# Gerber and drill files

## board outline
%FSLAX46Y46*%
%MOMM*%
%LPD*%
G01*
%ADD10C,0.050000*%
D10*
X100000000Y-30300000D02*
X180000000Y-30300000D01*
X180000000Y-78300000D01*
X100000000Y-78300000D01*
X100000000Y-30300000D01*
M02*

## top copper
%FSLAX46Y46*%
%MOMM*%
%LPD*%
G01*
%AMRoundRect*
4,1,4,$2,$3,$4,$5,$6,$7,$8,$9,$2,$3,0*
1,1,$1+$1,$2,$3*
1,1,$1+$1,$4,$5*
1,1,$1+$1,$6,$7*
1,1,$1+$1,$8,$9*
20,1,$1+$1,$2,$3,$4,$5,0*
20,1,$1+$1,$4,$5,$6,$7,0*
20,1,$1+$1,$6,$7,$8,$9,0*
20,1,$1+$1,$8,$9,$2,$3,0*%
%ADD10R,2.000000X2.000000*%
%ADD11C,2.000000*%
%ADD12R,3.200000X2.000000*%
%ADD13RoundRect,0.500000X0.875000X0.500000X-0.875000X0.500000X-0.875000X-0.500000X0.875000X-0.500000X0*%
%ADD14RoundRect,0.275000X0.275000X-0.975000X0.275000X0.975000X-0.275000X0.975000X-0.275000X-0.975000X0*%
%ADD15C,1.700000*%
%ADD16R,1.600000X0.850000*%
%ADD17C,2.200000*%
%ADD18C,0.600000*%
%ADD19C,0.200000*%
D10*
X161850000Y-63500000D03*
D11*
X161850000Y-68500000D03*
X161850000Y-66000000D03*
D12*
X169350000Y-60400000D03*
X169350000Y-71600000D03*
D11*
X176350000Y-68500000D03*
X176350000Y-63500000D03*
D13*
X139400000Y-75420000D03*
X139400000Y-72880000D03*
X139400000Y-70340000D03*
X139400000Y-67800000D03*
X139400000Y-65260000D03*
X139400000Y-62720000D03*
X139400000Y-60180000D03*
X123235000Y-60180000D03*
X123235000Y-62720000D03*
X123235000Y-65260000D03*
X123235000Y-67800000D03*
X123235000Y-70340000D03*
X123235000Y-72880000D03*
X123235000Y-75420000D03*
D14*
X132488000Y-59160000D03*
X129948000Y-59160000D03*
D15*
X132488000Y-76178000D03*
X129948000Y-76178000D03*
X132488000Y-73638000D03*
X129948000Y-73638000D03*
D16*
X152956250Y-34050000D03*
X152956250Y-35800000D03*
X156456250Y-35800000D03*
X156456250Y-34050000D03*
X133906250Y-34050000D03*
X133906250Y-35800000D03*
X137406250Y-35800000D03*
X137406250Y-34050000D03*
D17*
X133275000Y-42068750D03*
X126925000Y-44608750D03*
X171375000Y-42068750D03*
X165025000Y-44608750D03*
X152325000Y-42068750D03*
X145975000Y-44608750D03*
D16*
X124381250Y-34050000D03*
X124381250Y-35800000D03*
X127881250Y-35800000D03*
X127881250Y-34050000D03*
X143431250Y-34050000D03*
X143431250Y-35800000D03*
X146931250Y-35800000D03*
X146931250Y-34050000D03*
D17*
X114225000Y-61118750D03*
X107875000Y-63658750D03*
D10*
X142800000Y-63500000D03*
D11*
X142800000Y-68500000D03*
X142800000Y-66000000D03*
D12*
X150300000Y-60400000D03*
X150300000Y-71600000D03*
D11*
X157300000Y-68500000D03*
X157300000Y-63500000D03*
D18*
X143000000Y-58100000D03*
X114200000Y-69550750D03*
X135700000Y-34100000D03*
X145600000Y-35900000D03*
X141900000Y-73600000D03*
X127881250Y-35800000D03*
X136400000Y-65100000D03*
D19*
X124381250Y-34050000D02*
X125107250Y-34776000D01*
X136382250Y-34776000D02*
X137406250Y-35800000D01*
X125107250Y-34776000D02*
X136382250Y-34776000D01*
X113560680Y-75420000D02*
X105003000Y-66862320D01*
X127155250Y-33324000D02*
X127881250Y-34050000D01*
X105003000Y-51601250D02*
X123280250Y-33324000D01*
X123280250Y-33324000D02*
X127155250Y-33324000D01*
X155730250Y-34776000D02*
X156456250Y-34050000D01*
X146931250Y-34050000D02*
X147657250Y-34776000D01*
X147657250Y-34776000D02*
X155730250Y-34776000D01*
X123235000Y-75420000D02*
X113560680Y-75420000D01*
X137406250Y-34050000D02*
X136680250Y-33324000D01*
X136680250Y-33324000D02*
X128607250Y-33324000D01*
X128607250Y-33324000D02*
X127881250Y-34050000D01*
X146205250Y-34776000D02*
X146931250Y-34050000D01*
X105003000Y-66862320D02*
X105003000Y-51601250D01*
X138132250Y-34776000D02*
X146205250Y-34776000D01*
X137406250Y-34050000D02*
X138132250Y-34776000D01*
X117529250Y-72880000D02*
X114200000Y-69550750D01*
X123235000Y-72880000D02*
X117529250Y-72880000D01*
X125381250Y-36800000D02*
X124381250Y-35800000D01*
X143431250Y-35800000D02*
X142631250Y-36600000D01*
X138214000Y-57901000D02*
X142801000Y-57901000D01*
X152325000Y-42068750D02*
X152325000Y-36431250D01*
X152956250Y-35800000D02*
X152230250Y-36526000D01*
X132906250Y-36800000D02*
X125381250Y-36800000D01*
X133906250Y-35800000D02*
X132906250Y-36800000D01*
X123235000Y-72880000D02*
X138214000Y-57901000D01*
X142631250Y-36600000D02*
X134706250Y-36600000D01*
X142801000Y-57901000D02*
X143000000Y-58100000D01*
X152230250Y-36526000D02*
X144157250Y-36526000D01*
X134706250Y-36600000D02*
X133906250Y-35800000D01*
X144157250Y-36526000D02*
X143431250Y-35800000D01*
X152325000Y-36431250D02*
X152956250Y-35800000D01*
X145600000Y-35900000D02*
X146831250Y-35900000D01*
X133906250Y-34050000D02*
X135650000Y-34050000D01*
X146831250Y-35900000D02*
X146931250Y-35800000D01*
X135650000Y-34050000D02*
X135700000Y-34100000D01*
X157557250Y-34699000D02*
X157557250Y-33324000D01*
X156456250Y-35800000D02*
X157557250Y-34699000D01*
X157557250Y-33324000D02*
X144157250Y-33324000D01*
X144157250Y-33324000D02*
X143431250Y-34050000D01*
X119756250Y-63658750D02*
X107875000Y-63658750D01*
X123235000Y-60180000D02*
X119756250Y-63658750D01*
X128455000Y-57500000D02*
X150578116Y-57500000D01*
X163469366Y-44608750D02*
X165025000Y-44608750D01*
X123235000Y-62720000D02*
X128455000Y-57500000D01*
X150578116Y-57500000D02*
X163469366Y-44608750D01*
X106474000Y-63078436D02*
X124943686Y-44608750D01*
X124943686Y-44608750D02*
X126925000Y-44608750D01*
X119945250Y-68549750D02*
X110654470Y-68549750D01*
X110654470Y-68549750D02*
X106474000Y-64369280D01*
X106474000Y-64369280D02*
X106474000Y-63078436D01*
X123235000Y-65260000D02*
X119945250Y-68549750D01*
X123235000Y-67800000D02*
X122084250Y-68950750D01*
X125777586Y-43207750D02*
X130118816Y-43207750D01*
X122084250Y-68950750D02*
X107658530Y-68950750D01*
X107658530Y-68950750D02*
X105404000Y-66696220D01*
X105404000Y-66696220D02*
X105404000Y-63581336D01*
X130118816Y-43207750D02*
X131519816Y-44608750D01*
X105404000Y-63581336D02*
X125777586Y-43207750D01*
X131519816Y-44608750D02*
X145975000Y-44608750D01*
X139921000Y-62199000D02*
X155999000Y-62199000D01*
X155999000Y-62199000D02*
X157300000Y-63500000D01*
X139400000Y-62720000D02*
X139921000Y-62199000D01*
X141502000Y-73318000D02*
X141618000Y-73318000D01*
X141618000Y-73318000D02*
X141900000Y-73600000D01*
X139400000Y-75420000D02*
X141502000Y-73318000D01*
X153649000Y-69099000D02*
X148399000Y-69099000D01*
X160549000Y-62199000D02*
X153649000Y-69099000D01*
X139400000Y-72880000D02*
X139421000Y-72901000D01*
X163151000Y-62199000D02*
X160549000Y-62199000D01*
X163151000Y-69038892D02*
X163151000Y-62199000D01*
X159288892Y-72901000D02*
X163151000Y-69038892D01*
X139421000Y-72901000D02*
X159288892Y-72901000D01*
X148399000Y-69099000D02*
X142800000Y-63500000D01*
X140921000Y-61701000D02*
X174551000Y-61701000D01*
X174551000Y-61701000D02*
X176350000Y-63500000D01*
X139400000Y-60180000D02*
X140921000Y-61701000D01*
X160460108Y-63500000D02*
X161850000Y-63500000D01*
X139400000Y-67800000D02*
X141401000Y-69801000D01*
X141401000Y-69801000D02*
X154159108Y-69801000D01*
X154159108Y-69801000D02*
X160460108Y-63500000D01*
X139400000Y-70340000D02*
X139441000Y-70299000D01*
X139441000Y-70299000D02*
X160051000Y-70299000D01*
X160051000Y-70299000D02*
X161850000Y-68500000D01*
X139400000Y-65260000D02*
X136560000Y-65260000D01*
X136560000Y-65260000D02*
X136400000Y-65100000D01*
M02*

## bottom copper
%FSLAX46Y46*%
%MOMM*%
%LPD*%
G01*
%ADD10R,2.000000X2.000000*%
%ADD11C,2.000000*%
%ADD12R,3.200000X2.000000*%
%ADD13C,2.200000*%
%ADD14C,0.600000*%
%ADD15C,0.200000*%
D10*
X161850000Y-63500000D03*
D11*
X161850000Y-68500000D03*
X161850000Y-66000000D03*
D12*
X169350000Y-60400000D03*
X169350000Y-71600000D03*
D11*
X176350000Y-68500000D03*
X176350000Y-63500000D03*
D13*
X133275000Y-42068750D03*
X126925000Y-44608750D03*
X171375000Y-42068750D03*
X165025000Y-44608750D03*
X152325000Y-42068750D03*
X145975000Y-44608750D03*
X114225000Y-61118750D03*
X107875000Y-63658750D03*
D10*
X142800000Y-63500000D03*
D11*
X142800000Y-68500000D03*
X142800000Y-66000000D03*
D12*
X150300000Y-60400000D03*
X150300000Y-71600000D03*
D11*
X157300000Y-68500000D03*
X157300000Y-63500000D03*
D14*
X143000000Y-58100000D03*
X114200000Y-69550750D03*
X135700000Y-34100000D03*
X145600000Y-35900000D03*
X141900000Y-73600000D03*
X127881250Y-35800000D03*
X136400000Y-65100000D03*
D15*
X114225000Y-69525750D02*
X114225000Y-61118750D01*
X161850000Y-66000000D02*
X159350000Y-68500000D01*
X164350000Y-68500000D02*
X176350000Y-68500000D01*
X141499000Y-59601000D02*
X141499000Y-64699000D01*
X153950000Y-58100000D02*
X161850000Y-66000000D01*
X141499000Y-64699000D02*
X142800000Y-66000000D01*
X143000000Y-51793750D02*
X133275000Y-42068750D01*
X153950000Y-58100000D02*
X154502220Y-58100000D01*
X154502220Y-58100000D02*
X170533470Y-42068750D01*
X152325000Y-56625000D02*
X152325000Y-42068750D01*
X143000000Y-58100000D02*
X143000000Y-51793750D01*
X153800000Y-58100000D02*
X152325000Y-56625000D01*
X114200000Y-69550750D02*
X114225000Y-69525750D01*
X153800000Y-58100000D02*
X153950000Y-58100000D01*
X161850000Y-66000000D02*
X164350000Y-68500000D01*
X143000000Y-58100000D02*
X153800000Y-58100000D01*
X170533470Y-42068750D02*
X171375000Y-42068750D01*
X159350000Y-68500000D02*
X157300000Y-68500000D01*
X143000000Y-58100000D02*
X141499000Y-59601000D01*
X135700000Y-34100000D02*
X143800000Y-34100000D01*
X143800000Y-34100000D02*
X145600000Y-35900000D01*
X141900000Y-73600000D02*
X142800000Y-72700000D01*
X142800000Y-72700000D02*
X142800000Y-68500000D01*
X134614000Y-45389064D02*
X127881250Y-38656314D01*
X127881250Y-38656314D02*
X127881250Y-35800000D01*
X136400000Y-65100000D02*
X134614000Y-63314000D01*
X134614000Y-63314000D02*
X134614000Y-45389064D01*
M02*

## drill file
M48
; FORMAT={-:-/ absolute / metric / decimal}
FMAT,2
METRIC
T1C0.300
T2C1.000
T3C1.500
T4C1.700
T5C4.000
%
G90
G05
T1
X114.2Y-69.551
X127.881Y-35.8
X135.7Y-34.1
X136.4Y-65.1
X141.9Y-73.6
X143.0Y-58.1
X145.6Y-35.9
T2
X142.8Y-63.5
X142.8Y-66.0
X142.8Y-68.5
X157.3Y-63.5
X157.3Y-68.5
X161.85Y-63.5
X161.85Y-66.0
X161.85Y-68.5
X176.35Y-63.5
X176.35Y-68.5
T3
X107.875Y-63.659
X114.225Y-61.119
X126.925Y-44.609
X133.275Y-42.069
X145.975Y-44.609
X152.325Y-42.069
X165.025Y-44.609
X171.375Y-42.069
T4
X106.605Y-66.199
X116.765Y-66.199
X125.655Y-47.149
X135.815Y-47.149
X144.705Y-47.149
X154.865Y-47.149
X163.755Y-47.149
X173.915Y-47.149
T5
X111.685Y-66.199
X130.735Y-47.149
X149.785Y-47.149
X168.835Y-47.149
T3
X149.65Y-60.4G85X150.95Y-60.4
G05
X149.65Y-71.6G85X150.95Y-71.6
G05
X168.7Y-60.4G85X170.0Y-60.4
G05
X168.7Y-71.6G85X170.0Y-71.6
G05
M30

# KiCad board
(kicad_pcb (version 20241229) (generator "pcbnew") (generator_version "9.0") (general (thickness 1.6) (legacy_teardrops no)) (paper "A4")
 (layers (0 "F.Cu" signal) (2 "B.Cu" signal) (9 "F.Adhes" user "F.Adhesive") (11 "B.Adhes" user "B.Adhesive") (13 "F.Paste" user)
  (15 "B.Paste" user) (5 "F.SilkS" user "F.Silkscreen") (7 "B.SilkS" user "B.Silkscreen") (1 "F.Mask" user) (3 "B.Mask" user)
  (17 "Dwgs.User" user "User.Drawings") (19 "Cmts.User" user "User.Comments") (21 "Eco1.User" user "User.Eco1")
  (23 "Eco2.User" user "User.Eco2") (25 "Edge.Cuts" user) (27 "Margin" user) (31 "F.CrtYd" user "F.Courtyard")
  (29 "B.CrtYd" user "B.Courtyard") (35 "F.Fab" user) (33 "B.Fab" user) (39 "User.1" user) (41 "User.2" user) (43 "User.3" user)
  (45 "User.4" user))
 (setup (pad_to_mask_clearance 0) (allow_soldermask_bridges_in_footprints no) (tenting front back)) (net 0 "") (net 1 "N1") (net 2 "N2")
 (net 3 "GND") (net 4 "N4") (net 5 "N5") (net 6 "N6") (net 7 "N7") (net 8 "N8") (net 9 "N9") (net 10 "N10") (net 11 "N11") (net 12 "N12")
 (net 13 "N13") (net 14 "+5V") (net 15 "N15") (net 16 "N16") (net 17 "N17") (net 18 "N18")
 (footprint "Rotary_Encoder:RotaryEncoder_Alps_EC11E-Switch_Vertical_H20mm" (layer "F.Cu") (at 161.85 63.5)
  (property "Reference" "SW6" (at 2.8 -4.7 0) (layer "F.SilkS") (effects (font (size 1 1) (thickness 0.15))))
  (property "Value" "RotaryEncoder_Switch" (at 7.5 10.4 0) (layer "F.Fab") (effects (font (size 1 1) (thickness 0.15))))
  (pad "A" thru_hole rect (at 0 0) (size 2 2) (drill 1) (layers "*.Cu" "*.Mask") (remove_unused_layers no) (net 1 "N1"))
  (pad "B" thru_hole circle (at 0 5) (size 2 2) (drill 1) (layers "*.Cu" "*.Mask") (remove_unused_layers no) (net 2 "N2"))
  (pad "C" thru_hole circle (at 0 2.5) (size 2 2) (drill 1) (layers "*.Cu" "*.Mask") (remove_unused_layers no) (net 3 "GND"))
  (pad "MP" thru_hole rect (at 7.5 -3.1) (size 3.2 2) (drill oval 2.8 1.5) (layers "*.Cu" "*.Mask") (remove_unused_layers no))
  (pad "MP" thru_hole rect (at 7.5 8.1) (size 3.2 2) (drill oval 2.8 1.5) (layers "*.Cu" "*.Mask") (remove_unused_layers no))
  (pad "S1" thru_hole circle (at 14.5 5) (size 2 2) (drill 1) (layers "*.Cu" "*.Mask") (remove_unused_layers no) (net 3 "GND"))
  (pad "S2" thru_hole circle (at 14.5 0) (size 2 2) (drill 1) (layers "*.Cu" "*.Mask") (remove_unused_layers no) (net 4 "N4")))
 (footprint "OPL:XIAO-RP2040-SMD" (layer "F.Cu") (at 131.4 67.8 180)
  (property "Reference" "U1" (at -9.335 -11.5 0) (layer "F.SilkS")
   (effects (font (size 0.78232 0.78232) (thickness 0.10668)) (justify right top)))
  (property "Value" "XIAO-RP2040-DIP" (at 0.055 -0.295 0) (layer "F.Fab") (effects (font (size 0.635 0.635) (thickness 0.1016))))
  (pad "1" smd roundrect (at -8 -7.62 180) (size 2.75 2) (layers "F.Cu" "F.Mask" "F.Paste") (roundrect_rratio 0.25) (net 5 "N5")
   (solder_mask_margin 0.0508) (thermal_bridge_angle 45))
  (pad "2" smd roundrect (at -8 -5.08 180) (size 2.75 2) (layers "F.Cu" "F.Mask" "F.Paste") (roundrect_rratio 0.25) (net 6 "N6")
   (solder_mask_margin 0.0508) (thermal_bridge_angle 45))
  (pad "3" smd roundrect (at -8 -2.54 180) (size 2.75 2) (layers "F.Cu" "F.Mask" "F.Paste") (roundrect_rratio 0.25) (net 2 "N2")
   (solder_mask_margin 0.0508) (thermal_bridge_angle 45))
  (pad "4" smd roundrect (at -8 0 180) (size 2.75 2) (layers "F.Cu" "F.Mask" "F.Paste") (roundrect_rratio 0.25) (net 1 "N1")
   (solder_mask_margin 0.0508) (thermal_bridge_angle 45))
  (pad "5" smd roundrect (at -8 2.54 180) (size 2.75 2) (layers "F.Cu" "F.Mask" "F.Paste") (roundrect_rratio 0.25) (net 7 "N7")
   (solder_mask_margin 0.0508) (thermal_bridge_angle 45))
  (pad "6" smd roundrect (at -8 5.08 180) (size 2.75 2) (layers "F.Cu" "F.Mask" "F.Paste") (roundrect_rratio 0.25) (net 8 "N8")
   (solder_mask_margin 0.0508) (thermal_bridge_angle 45))
  (pad "7" smd roundrect (at -8 7.62 180) (size 2.75 2) (layers "F.Cu" "F.Mask" "F.Paste") (roundrect_rratio 0.25) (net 4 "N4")
   (solder_mask_margin 0.0508) (thermal_bridge_angle 45))
  (pad "8" smd roundrect (at 8.165 7.62 180) (size 2.75 2) (layers "F.Cu" "F.Mask" "F.Paste") (roundrect_rratio 0.25) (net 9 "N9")
   (solder_mask_margin 0.0508) (thermal_bridge_angle 45))
  (pad "9" smd roundrect (at 8.165 5.08 180) (size 2.75 2) (layers "F.Cu" "F.Mask" "F.Paste") (roundrect_rratio 0.25) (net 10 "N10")
   (solder_mask_margin 0.0508) (thermal_bridge_angle 45))
  (pad "10" smd roundrect (at 8.165 2.54 180) (size 2.75 2) (layers "F.Cu" "F.Mask" "F.Paste") (roundrect_rratio 0.25) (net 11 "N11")
   (solder_mask_margin 0.0508) (thermal_bridge_angle 45))
  (pad "11" smd roundrect (at 8.165 0 180) (size 2.75 2) (layers "F.Cu" "F.Mask" "F.Paste") (roundrect_rratio 0.25) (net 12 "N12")
   (solder_mask_margin 0.0508) (thermal_bridge_angle 45))
  (pad "12" smd roundrect (at 8.165 -2.54 180) (size 2.75 2) (layers "F.Cu" "F.Mask" "F.Paste") (roundrect_rratio 0.25) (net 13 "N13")
   (solder_mask_margin 0.0508) (thermal_bridge_angle 45))
  (pad "13" smd roundrect (at 8.165 -5.08 180) (size 2.75 2) (layers "F.Cu" "F.Mask" "F.Paste") (roundrect_rratio 0.25) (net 3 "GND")
   (solder_mask_margin 0.0508) (thermal_bridge_angle 45))
  (pad "14" smd roundrect (at 8.165 -7.62 180) (size 2.75 2) (layers "F.Cu" "F.Mask" "F.Paste") (roundrect_rratio 0.25) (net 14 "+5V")
   (solder_mask_margin 0.0508) (thermal_bridge_angle 45))
  (pad "15" smd roundrect (at -1.088 8.64 90) (size 2.5 1.1) (layers "F.Cu" "F.Mask" "F.Paste") (roundrect_rratio 0.25)
   (thermal_bridge_angle 45))
  (pad "16" smd roundrect (at 1.452 8.64 90) (size 2.5 1.1) (layers "F.Cu" "F.Mask" "F.Paste") (roundrect_rratio 0.25)
   (thermal_bridge_angle 45))
  (pad "17" smd circle (at -1.088 -8.378 180) (size 1.7 1.7) (layers "F.Cu" "F.Mask" "F.Paste"))
  (pad "18" smd circle (at 1.452 -8.378 180) (size 1.7 1.7) (layers "F.Cu" "F.Mask" "F.Paste"))
  (pad "19" smd circle (at -1.088 -5.838 180) (size 1.7 1.7) (layers "F.Cu" "F.Mask" "F.Paste"))
  (pad "20" smd circle (at 1.452 -5.838 180) (size 1.7 1.7) (layers "F.Cu" "F.Mask" "F.Paste")))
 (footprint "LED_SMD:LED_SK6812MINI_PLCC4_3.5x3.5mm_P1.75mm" (layer "F.Cu") (at 154.70625 34.925)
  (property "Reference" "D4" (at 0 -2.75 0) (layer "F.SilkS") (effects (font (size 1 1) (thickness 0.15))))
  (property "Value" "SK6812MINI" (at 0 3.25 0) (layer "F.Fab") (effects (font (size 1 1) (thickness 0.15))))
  (pad "1" smd rect (at -1.75 -0.875) (size 1.6 0.85) (layers "F.Cu" "F.Mask" "F.Paste") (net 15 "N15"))
  (pad "2" smd rect (at -1.75 0.875) (size 1.6 0.85) (layers "F.Cu" "F.Mask" "F.Paste") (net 3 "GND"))
  (pad "3" smd rect (at 1.75 0.875) (size 1.6 0.85) (layers "F.Cu" "F.Mask" "F.Paste") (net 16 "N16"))
  (pad "4" smd rect (at 1.75 -0.875) (size 1.6 0.85) (layers "F.Cu" "F.Mask" "F.Paste") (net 14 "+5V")))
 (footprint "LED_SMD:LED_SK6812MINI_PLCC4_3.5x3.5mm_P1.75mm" (layer "F.Cu") (at 135.65625 34.925)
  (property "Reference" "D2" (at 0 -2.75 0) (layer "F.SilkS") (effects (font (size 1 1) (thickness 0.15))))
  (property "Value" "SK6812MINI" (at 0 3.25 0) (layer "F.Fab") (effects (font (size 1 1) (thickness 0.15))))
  (pad "1" smd rect (at -1.75 -0.875) (size 1.6 0.85) (layers "F.Cu" "F.Mask" "F.Paste") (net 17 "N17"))
  (pad "2" smd rect (at -1.75 0.875) (size 1.6 0.85) (layers "F.Cu" "F.Mask" "F.Paste") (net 3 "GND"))
  (pad "3" smd rect (at 1.75 0.875) (size 1.6 0.85) (layers "F.Cu" "F.Mask" "F.Paste") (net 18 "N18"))
  (pad "4" smd rect (at 1.75 -0.875) (size 1.6 0.85) (layers "F.Cu" "F.Mask" "F.Paste") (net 14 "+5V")))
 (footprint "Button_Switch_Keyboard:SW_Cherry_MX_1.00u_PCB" (layer "F.Cu") (at 133.275 42.06875)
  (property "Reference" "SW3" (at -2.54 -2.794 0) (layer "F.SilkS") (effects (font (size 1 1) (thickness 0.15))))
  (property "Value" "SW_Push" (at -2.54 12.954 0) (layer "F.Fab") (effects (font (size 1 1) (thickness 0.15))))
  (pad "" np_thru_hole circle (at -7.62 5.08) (size 1.7 1.7) (drill 1.7) (layers "*.Cu" "*.Mask"))
  (pad "" np_thru_hole circle (at -2.54 5.08) (size 4 4) (drill 4) (layers "*.Cu" "*.Mask"))
  (pad "" np_thru_hole circle (at 2.54 5.08) (size 1.7 1.7) (drill 1.7) (layers "*.Cu" "*.Mask"))
  (pad "1" thru_hole circle (at 0 0) (size 2.2 2.2) (drill 1.5) (layers "*.Cu" "*.Mask") (remove_unused_layers no) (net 3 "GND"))
  (pad "2" thru_hole circle (at -6.35 2.54) (size 2.2 2.2) (drill 1.5) (layers "*.Cu" "*.Mask") (remove_unused_layers no) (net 11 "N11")))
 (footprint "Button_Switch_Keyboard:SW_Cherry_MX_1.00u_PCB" (layer "F.Cu") (at 171.375 42.06875)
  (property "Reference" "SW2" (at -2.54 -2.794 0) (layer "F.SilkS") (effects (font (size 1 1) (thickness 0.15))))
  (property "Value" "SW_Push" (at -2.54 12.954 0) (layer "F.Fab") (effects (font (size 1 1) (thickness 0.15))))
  (pad "" np_thru_hole circle (at -7.62 5.08) (size 1.7 1.7) (drill 1.7) (layers "*.Cu" "*.Mask"))
  (pad "" np_thru_hole circle (at -2.54 5.08) (size 4 4) (drill 4) (layers "*.Cu" "*.Mask"))
  (pad "" np_thru_hole circle (at 2.54 5.08) (size 1.7 1.7) (drill 1.7) (layers "*.Cu" "*.Mask"))
  (pad "1" thru_hole circle (at 0 0) (size 2.2 2.2) (drill 1.5) (layers "*.Cu" "*.Mask") (remove_unused_layers no) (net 3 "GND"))
  (pad "2" thru_hole circle (at -6.35 2.54) (size 2.2 2.2) (drill 1.5) (layers "*.Cu" "*.Mask") (remove_unused_layers no) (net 10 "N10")))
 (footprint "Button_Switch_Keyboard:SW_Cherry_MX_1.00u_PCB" (layer "F.Cu") (at 152.325 42.06875)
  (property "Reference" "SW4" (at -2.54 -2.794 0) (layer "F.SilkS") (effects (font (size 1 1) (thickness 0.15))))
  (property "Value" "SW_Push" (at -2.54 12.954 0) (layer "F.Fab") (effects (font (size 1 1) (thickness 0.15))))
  (pad "" np_thru_hole circle (at -7.62 5.08) (size 1.7 1.7) (drill 1.7) (layers "*.Cu" "*.Mask"))
  (pad "" np_thru_hole circle (at -2.54 5.08) (size 4 4) (drill 4) (layers "*.Cu" "*.Mask"))
  (pad "" np_thru_hole circle (at 2.54 5.08) (size 1.7 1.7) (drill 1.7) (layers "*.Cu" "*.Mask"))
  (pad "1" thru_hole circle (at 0 0) (size 2.2 2.2) (drill 1.5) (layers "*.Cu" "*.Mask") (remove_unused_layers no) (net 3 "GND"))
  (pad "2" thru_hole circle (at -6.35 2.54) (size 2.2 2.2) (drill 1.5) (layers "*.Cu" "*.Mask") (remove_unused_layers no) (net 12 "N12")))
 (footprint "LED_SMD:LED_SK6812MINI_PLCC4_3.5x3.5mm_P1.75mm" (layer "F.Cu") (at 126.13125 34.925)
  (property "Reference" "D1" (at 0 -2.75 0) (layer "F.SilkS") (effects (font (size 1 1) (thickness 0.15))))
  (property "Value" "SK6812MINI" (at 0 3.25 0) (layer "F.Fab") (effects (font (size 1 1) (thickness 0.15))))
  (pad "1" smd rect (at -1.75 -0.875) (size 1.6 0.85) (layers "F.Cu" "F.Mask" "F.Paste") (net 18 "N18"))
  (pad "2" smd rect (at -1.75 0.875) (size 1.6 0.85) (layers "F.Cu" "F.Mask" "F.Paste") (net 3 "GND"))
  (pad "3" smd rect (at 1.75 0.875) (size 1.6 0.85) (layers "F.Cu" "F.Mask" "F.Paste") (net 7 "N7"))
  (pad "4" smd rect (at 1.75 -0.875) (size 1.6 0.85) (layers "F.Cu" "F.Mask" "F.Paste") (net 14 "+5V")))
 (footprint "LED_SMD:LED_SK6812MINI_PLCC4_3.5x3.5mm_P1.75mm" (layer "F.Cu") (at 145.18125 34.925)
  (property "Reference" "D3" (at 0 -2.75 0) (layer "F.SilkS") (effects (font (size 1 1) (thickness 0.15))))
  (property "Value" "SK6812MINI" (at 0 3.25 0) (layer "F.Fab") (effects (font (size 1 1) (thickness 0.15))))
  (pad "1" smd rect (at -1.75 -0.875) (size 1.6 0.85) (layers "F.Cu" "F.Mask" "F.Paste") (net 16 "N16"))
  (pad "2" smd rect (at -1.75 0.875) (size 1.6 0.85) (layers "F.Cu" "F.Mask" "F.Paste") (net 3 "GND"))
  (pad "3" smd rect (at 1.75 0.875) (size 1.6 0.85) (layers "F.Cu" "F.Mask" "F.Paste") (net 17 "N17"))
  (pad "4" smd rect (at 1.75 -0.875) (size 1.6 0.85) (layers "F.Cu" "F.Mask" "F.Paste") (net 14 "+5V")))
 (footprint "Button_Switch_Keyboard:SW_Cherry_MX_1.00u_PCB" (layer "F.Cu") (at 114.225 61.11875)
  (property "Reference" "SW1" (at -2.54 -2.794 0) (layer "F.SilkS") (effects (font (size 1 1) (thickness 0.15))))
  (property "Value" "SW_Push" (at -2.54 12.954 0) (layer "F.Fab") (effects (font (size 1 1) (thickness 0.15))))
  (pad "" np_thru_hole circle (at -7.62 5.08) (size 1.7 1.7) (drill 1.7) (layers "*.Cu" "*.Mask"))
  (pad "" np_thru_hole circle (at -2.54 5.08) (size 4 4) (drill 4) (layers "*.Cu" "*.Mask"))
  (pad "" np_thru_hole circle (at 2.54 5.08) (size 1.7 1.7) (drill 1.7) (layers "*.Cu" "*.Mask"))
  (pad "1" thru_hole circle (at 0 0) (size 2.2 2.2) (drill 1.5) (layers "*.Cu" "*.Mask") (remove_unused_layers no) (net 3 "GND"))
  (pad "2" thru_hole circle (at -6.35 2.54) (size 2.2 2.2) (drill 1.5) (layers "*.Cu" "*.Mask") (remove_unused_layers no) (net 9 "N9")))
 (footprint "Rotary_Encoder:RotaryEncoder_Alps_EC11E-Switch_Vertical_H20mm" (layer "F.Cu") (at 142.8 63.5)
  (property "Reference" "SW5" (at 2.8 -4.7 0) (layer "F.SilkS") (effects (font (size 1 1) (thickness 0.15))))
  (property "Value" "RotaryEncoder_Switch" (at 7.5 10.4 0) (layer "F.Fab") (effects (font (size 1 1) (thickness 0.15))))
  (pad "A" thru_hole rect (at 0 0) (size 2 2) (drill 1) (layers "*.Cu" "*.Mask") (remove_unused_layers no) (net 6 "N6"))
  (pad "B" thru_hole circle (at 0 5) (size 2 2) (drill 1) (layers "*.Cu" "*.Mask") (remove_unused_layers no) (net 5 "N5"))
  (pad "C" thru_hole circle (at 0 2.5) (size 2 2) (drill 1) (layers "*.Cu" "*.Mask") (remove_unused_layers no) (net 3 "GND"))
  (pad "MP" thru_hole rect (at 7.5 -3.1) (size 3.2 2) (drill oval 2.8 1.5) (layers "*.Cu" "*.Mask") (remove_unused_layers no))
  (pad "MP" thru_hole rect (at 7.5 8.1) (size 3.2 2) (drill oval 2.8 1.5) (layers "*.Cu" "*.Mask") (remove_unused_layers no))
  (pad "S1" thru_hole circle (at 14.5 5) (size 2 2) (drill 1) (layers "*.Cu" "*.Mask") (remove_unused_layers no) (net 3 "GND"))
  (pad "S2" thru_hole circle (at 14.5 0) (size 2 2) (drill 1) (layers "*.Cu" "*.Mask") (remove_unused_layers no) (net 8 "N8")))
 (gr_rect (start 100 30.3) (end 180 78.3) (stroke (width 0.05) (type solid)) (fill no) (layer "Edge.Cuts"))
 (segment (start 124.38125 34.05) (end 125.10725 34.776) (width 0.2) (layer "F.Cu") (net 18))
 (segment (start 136.38225 34.776) (end 137.40625 35.8) (width 0.2) (layer "F.Cu") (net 18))
 (segment (start 125.10725 34.776) (end 136.38225 34.776) (width 0.2) (layer "F.Cu") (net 18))
 (segment (start 113.56068 75.42) (end 105.003 66.86232) (width 0.2) (layer "F.Cu") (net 14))
 (segment (start 127.15525 33.324) (end 127.88125 34.05) (width 0.2) (layer "F.Cu") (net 14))
 (segment (start 105.003 51.60125) (end 123.28025 33.324) (width 0.2) (layer "F.Cu") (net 14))
 (segment (start 123.28025 33.324) (end 127.15525 33.324) (width 0.2) (layer "F.Cu") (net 14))
 (segment (start 155.73025 34.776) (end 156.45625 34.05) (width 0.2) (layer "F.Cu") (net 14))
 (segment (start 146.93125 34.05) (end 147.65725 34.776) (width 0.2) (layer "F.Cu") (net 14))
 (segment (start 147.65725 34.776) (end 155.73025 34.776) (width 0.2) (layer "F.Cu") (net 14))
 (segment (start 123.235 75.42) (end 113.56068 75.42) (width 0.2) (layer "F.Cu") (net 14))
 (segment (start 137.40625 34.05) (end 136.68025 33.324) (width 0.2) (layer "F.Cu") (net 14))
 (segment (start 136.68025 33.324) (end 128.60725 33.324) (width 0.2) (layer "F.Cu") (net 14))
 (segment (start 128.60725 33.324) (end 127.88125 34.05) (width 0.2) (layer "F.Cu") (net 14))
 (segment (start 146.20525 34.776) (end 146.93125 34.05) (width 0.2) (layer "F.Cu") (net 14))
 (segment (start 105.003 66.86232) (end 105.003 51.60125) (width 0.2) (layer "F.Cu") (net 14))
 (segment (start 138.13225 34.776) (end 146.20525 34.776) (width 0.2) (layer "F.Cu") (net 14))
 (segment (start 137.40625 34.05) (end 138.13225 34.776) (width 0.2) (layer "F.Cu") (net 14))
 (segment (start 117.52925 72.88) (end 114.2 69.55075) (width 0.2) (layer "F.Cu") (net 3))
 (segment (start 123.235 72.88) (end 117.52925 72.88) (width 0.2) (layer "F.Cu") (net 3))
 (segment (start 125.38125 36.8) (end 124.38125 35.8) (width 0.2) (layer "F.Cu") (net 3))
 (segment (start 143.43125 35.8) (end 142.63125 36.6) (width 0.2) (layer "F.Cu") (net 3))
 (segment (start 138.214 57.901) (end 142.801 57.901) (width 0.2) (layer "F.Cu") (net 3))
 (segment (start 152.325 42.06875) (end 152.325 36.43125) (width 0.2) (layer "F.Cu") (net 3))
 (segment (start 152.95625 35.8) (end 152.23025 36.526) (width 0.2) (layer "F.Cu") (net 3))
 (segment (start 132.90625 36.8) (end 125.38125 36.8) (width 0.2) (layer "F.Cu") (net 3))
 (segment (start 133.90625 35.8) (end 132.90625 36.8) (width 0.2) (layer "F.Cu") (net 3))
 (segment (start 123.235 72.88) (end 138.214 57.901) (width 0.2) (layer "F.Cu") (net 3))
 (segment (start 142.63125 36.6) (end 134.70625 36.6) (width 0.2) (layer "F.Cu") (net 3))
 (segment (start 142.801 57.901) (end 143 58.1) (width 0.2) (layer "F.Cu") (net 3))
 (segment (start 152.23025 36.526) (end 144.15725 36.526) (width 0.2) (layer "F.Cu") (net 3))
 (segment (start 134.70625 36.6) (end 133.90625 35.8) (width 0.2) (layer "F.Cu") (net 3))
 (segment (start 144.15725 36.526) (end 143.43125 35.8) (width 0.2) (layer "F.Cu") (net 3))
 (segment (start 152.325 36.43125) (end 152.95625 35.8) (width 0.2) (layer "F.Cu") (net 3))
 (via (at 143 58.1) (size 0.6) (drill 0.3) (layers "F.Cu" "B.Cu") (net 3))
 (via (at 114.2 69.55075) (size 0.6) (drill 0.3) (layers "F.Cu" "B.Cu") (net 3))
 (segment (start 114.225 69.52575) (end 114.225 61.11875) (width 0.2) (layer "B.Cu") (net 3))
 (segment (start 161.85 66) (end 159.35 68.5) (width 0.2) (layer "B.Cu") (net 3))
 (segment (start 164.35 68.5) (end 176.35 68.5) (width 0.2) (layer "B.Cu") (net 3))
 (segment (start 141.499 59.601) (end 141.499 64.699) (width 0.2) (layer "B.Cu") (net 3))
 (segment (start 153.95 58.1) (end 161.85 66) (width 0.2) (layer "B.Cu") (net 3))
 (segment (start 141.499 64.699) (end 142.8 66) (width 0.2) (layer "B.Cu") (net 3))
 (segment (start 143 51.79375) (end 133.275 42.06875) (width 0.2) (layer "B.Cu") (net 3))
 (segment (start 153.95 58.1) (end 154.50222 58.1) (width 0.2) (layer "B.Cu") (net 3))
 (segment (start 154.50222 58.1) (end 170.53347 42.06875) (width 0.2) (layer "B.Cu") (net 3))
 (segment (start 152.325 56.625) (end 152.325 42.06875) (width 0.2) (layer "B.Cu") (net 3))
 (segment (start 143 58.1) (end 143 51.79375) (width 0.2) (layer "B.Cu") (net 3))
 (segment (start 153.8 58.1) (end 152.325 56.625) (width 0.2) (layer "B.Cu") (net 3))
 (segment (start 114.2 69.55075) (end 114.225 69.52575) (width 0.2) (layer "B.Cu") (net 3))
 (segment (start 153.8 58.1) (end 153.95 58.1) (width 0.2) (layer "B.Cu") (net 3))
 (segment (start 161.85 66) (end 164.35 68.5) (width 0.2) (layer "B.Cu") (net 3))
 (segment (start 143 58.1) (end 153.8 58.1) (width 0.2) (layer "B.Cu") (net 3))
 (segment (start 170.53347 42.06875) (end 171.375 42.06875) (width 0.2) (layer "B.Cu") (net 3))
 (segment (start 159.35 68.5) (end 157.3 68.5) (width 0.2) (layer "B.Cu") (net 3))
 (segment (start 143 58.1) (end 141.499 59.601) (width 0.2) (layer "B.Cu") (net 3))
 (segment (start 145.6 35.9) (end 146.83125 35.9) (width 0.2) (layer "F.Cu") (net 17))
 (segment (start 133.90625 34.05) (end 135.65 34.05) (width 0.2) (layer "F.Cu") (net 17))
 (segment (start 146.83125 35.9) (end 146.93125 35.8) (width 0.2) (layer "F.Cu") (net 17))
 (segment (start 135.65 34.05) (end 135.7 34.1) (width 0.2) (layer "F.Cu") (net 17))
 (via (at 135.7 34.1) (size 0.6) (drill 0.3) (layers "F.Cu" "B.Cu") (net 17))
 (via (at 145.6 35.9) (size 0.6) (drill 0.3) (layers "F.Cu" "B.Cu") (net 17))
 (segment (start 135.7 34.1) (end 143.8 34.1) (width 0.2) (layer "B.Cu") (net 17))
 (segment (start 143.8 34.1) (end 145.6 35.9) (width 0.2) (layer "B.Cu") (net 17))
 (segment (start 157.55725 34.699) (end 157.55725 33.324) (width 0.2) (layer "F.Cu") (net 16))
 (segment (start 156.45625 35.8) (end 157.55725 34.699) (width 0.2) (layer "F.Cu") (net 16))
 (segment (start 157.55725 33.324) (end 144.15725 33.324) (width 0.2) (layer "F.Cu") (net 16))
 (segment (start 144.15725 33.324) (end 143.43125 34.05) (width 0.2) (layer "F.Cu") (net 16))
 (segment (start 119.75625 63.65875) (end 107.875 63.65875) (width 0.2) (layer "F.Cu") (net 9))
 (segment (start 123.235 60.18) (end 119.75625 63.65875) (width 0.2) (layer "F.Cu") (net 9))
 (segment (start 128.455 57.5) (end 150.578116 57.5) (width 0.2) (layer "F.Cu") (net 10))
 (segment (start 163.469366 44.60875) (end 165.025 44.60875) (width 0.2) (layer "F.Cu") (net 10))
 (segment (start 123.235 62.72) (end 128.455 57.5) (width 0.2) (layer "F.Cu") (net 10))
 (segment (start 150.578116 57.5) (end 163.469366 44.60875) (width 0.2) (layer "F.Cu") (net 10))
 (segment (start 106.474 63.078436) (end 124.943686 44.60875) (width 0.2) (layer "F.Cu") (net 11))
 (segment (start 124.943686 44.60875) (end 126.925 44.60875) (width 0.2) (layer "F.Cu") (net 11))
 (segment (start 119.94525 68.54975) (end 110.65447 68.54975) (width 0.2) (layer "F.Cu") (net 11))
 (segment (start 110.65447 68.54975) (end 106.474 64.36928) (width 0.2) (layer "F.Cu") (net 11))
 (segment (start 106.474 64.36928) (end 106.474 63.078436) (width 0.2) (layer "F.Cu") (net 11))
 (segment (start 123.235 65.26) (end 119.94525 68.54975) (width 0.2) (layer "F.Cu") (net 11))
 (segment (start 123.235 67.8) (end 122.08425 68.95075) (width 0.2) (layer "F.Cu") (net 12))
 (segment (start 125.777586 43.20775) (end 130.118816 43.20775) (width 0.2) (layer "F.Cu") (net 12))
 (segment (start 122.08425 68.95075) (end 107.65853 68.95075) (width 0.2) (layer "F.Cu") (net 12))
 (segment (start 107.65853 68.95075) (end 105.404 66.69622) (width 0.2) (layer "F.Cu") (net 12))
 (segment (start 105.404 66.69622) (end 105.404 63.581336) (width 0.2) (layer "F.Cu") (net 12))
 (segment (start 130.118816 43.20775) (end 131.519816 44.60875) (width 0.2) (layer "F.Cu") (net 12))
 (segment (start 105.404 63.581336) (end 125.777586 43.20775) (width 0.2) (layer "F.Cu") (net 12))
 (segment (start 131.519816 44.60875) (end 145.975 44.60875) (width 0.2) (layer "F.Cu") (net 12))
 (segment (start 139.921 62.199) (end 155.999 62.199) (width 0.2) (layer "F.Cu") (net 8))
 (segment (start 155.999 62.199) (end 157.3 63.5) (width 0.2) (layer "F.Cu") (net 8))
 (segment (start 139.4 62.72) (end 139.921 62.199) (width 0.2) (layer "F.Cu") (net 8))
 (segment (start 141.502 73.318) (end 141.618 73.318) (width 0.2) (layer "F.Cu") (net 5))
 (segment (start 141.618 73.318) (end 141.9 73.6) (width 0.2) (layer "F.Cu") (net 5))
 (segment (start 139.4 75.42) (end 141.502 73.318) (width 0.2) (layer "F.Cu") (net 5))
 (via (at 141.9 73.6) (size 0.6) (drill 0.3) (layers "F.Cu" "B.Cu") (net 5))
 (segment (start 141.9 73.6) (end 142.8 72.7) (width 0.2) (layer "B.Cu") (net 5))
 (segment (start 142.8 72.7) (end 142.8 68.5) (width 0.2) (layer "B.Cu") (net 5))
 (segment (start 153.649 69.099) (end 148.399 69.099) (width 0.2) (layer "F.Cu") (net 6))
 (segment (start 160.549 62.199) (end 153.649 69.099) (width 0.2) (layer "F.Cu") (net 6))
 (segment (start 139.4 72.88) (end 139.421 72.901) (width 0.2) (layer "F.Cu") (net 6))
 (segment (start 163.151 62.199) (end 160.549 62.199) (width 0.2) (layer "F.Cu") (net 6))
 (segment (start 163.151 69.038892) (end 163.151 62.199) (width 0.2) (layer "F.Cu") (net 6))
 (segment (start 159.288892 72.901) (end 163.151 69.038892) (width 0.2) (layer "F.Cu") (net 6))
 (segment (start 139.421 72.901) (end 159.288892 72.901) (width 0.2) (layer "F.Cu") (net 6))
 (segment (start 148.399 69.099) (end 142.8 63.5) (width 0.2) (layer "F.Cu") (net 6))
 (segment (start 140.921 61.701) (end 174.551 61.701) (width 0.2) (layer "F.Cu") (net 4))
 (segment (start 174.551 61.701) (end 176.35 63.5) (width 0.2) (layer "F.Cu") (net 4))
 (segment (start 139.4 60.18) (end 140.921 61.701) (width 0.2) (layer "F.Cu") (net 4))
 (segment (start 160.460108 63.5) (end 161.85 63.5) (width 0.2) (layer "F.Cu") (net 1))
 (segment (start 139.4 67.8) (end 141.401 69.801) (width 0.2) (layer "F.Cu") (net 1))
 (segment (start 141.401 69.801) (end 154.159108 69.801) (width 0.2) (layer "F.Cu") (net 1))
 (segment (start 154.159108 69.801) (end 160.460108 63.5) (width 0.2) (layer "F.Cu") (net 1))
 (segment (start 139.4 70.34) (end 139.441 70.299) (width 0.2) (layer "F.Cu") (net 2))
 (segment (start 139.441 70.299) (end 160.051 70.299) (width 0.2) (layer "F.Cu") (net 2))
 (segment (start 160.051 70.299) (end 161.85 68.5) (width 0.2) (layer "F.Cu") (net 2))
 (segment (start 139.4 65.26) (end 136.56 65.26) (width 0.2) (layer "F.Cu") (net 7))
 (segment (start 136.56 65.26) (end 136.4 65.1) (width 0.2) (layer "F.Cu") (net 7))
 (via (at 127.88125 35.8) (size 0.6) (drill 0.3) (layers "F.Cu" "B.Cu") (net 7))
 (via (at 136.4 65.1) (size 0.6) (drill 0.3) (layers "F.Cu" "B.Cu") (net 7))
 (segment (start 134.614 45.389064) (end 127.88125 38.656314) (width 0.2) (layer "B.Cu") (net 7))
 (segment (start 127.88125 38.656314) (end 127.88125 35.8) (width 0.2) (layer "B.Cu") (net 7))
 (segment (start 136.4 65.1) (end 134.614 63.314) (width 0.2) (layer "B.Cu") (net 7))
 (segment (start 134.614 63.314) (end 134.614 45.389064) (width 0.2) (layer "B.Cu") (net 7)))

